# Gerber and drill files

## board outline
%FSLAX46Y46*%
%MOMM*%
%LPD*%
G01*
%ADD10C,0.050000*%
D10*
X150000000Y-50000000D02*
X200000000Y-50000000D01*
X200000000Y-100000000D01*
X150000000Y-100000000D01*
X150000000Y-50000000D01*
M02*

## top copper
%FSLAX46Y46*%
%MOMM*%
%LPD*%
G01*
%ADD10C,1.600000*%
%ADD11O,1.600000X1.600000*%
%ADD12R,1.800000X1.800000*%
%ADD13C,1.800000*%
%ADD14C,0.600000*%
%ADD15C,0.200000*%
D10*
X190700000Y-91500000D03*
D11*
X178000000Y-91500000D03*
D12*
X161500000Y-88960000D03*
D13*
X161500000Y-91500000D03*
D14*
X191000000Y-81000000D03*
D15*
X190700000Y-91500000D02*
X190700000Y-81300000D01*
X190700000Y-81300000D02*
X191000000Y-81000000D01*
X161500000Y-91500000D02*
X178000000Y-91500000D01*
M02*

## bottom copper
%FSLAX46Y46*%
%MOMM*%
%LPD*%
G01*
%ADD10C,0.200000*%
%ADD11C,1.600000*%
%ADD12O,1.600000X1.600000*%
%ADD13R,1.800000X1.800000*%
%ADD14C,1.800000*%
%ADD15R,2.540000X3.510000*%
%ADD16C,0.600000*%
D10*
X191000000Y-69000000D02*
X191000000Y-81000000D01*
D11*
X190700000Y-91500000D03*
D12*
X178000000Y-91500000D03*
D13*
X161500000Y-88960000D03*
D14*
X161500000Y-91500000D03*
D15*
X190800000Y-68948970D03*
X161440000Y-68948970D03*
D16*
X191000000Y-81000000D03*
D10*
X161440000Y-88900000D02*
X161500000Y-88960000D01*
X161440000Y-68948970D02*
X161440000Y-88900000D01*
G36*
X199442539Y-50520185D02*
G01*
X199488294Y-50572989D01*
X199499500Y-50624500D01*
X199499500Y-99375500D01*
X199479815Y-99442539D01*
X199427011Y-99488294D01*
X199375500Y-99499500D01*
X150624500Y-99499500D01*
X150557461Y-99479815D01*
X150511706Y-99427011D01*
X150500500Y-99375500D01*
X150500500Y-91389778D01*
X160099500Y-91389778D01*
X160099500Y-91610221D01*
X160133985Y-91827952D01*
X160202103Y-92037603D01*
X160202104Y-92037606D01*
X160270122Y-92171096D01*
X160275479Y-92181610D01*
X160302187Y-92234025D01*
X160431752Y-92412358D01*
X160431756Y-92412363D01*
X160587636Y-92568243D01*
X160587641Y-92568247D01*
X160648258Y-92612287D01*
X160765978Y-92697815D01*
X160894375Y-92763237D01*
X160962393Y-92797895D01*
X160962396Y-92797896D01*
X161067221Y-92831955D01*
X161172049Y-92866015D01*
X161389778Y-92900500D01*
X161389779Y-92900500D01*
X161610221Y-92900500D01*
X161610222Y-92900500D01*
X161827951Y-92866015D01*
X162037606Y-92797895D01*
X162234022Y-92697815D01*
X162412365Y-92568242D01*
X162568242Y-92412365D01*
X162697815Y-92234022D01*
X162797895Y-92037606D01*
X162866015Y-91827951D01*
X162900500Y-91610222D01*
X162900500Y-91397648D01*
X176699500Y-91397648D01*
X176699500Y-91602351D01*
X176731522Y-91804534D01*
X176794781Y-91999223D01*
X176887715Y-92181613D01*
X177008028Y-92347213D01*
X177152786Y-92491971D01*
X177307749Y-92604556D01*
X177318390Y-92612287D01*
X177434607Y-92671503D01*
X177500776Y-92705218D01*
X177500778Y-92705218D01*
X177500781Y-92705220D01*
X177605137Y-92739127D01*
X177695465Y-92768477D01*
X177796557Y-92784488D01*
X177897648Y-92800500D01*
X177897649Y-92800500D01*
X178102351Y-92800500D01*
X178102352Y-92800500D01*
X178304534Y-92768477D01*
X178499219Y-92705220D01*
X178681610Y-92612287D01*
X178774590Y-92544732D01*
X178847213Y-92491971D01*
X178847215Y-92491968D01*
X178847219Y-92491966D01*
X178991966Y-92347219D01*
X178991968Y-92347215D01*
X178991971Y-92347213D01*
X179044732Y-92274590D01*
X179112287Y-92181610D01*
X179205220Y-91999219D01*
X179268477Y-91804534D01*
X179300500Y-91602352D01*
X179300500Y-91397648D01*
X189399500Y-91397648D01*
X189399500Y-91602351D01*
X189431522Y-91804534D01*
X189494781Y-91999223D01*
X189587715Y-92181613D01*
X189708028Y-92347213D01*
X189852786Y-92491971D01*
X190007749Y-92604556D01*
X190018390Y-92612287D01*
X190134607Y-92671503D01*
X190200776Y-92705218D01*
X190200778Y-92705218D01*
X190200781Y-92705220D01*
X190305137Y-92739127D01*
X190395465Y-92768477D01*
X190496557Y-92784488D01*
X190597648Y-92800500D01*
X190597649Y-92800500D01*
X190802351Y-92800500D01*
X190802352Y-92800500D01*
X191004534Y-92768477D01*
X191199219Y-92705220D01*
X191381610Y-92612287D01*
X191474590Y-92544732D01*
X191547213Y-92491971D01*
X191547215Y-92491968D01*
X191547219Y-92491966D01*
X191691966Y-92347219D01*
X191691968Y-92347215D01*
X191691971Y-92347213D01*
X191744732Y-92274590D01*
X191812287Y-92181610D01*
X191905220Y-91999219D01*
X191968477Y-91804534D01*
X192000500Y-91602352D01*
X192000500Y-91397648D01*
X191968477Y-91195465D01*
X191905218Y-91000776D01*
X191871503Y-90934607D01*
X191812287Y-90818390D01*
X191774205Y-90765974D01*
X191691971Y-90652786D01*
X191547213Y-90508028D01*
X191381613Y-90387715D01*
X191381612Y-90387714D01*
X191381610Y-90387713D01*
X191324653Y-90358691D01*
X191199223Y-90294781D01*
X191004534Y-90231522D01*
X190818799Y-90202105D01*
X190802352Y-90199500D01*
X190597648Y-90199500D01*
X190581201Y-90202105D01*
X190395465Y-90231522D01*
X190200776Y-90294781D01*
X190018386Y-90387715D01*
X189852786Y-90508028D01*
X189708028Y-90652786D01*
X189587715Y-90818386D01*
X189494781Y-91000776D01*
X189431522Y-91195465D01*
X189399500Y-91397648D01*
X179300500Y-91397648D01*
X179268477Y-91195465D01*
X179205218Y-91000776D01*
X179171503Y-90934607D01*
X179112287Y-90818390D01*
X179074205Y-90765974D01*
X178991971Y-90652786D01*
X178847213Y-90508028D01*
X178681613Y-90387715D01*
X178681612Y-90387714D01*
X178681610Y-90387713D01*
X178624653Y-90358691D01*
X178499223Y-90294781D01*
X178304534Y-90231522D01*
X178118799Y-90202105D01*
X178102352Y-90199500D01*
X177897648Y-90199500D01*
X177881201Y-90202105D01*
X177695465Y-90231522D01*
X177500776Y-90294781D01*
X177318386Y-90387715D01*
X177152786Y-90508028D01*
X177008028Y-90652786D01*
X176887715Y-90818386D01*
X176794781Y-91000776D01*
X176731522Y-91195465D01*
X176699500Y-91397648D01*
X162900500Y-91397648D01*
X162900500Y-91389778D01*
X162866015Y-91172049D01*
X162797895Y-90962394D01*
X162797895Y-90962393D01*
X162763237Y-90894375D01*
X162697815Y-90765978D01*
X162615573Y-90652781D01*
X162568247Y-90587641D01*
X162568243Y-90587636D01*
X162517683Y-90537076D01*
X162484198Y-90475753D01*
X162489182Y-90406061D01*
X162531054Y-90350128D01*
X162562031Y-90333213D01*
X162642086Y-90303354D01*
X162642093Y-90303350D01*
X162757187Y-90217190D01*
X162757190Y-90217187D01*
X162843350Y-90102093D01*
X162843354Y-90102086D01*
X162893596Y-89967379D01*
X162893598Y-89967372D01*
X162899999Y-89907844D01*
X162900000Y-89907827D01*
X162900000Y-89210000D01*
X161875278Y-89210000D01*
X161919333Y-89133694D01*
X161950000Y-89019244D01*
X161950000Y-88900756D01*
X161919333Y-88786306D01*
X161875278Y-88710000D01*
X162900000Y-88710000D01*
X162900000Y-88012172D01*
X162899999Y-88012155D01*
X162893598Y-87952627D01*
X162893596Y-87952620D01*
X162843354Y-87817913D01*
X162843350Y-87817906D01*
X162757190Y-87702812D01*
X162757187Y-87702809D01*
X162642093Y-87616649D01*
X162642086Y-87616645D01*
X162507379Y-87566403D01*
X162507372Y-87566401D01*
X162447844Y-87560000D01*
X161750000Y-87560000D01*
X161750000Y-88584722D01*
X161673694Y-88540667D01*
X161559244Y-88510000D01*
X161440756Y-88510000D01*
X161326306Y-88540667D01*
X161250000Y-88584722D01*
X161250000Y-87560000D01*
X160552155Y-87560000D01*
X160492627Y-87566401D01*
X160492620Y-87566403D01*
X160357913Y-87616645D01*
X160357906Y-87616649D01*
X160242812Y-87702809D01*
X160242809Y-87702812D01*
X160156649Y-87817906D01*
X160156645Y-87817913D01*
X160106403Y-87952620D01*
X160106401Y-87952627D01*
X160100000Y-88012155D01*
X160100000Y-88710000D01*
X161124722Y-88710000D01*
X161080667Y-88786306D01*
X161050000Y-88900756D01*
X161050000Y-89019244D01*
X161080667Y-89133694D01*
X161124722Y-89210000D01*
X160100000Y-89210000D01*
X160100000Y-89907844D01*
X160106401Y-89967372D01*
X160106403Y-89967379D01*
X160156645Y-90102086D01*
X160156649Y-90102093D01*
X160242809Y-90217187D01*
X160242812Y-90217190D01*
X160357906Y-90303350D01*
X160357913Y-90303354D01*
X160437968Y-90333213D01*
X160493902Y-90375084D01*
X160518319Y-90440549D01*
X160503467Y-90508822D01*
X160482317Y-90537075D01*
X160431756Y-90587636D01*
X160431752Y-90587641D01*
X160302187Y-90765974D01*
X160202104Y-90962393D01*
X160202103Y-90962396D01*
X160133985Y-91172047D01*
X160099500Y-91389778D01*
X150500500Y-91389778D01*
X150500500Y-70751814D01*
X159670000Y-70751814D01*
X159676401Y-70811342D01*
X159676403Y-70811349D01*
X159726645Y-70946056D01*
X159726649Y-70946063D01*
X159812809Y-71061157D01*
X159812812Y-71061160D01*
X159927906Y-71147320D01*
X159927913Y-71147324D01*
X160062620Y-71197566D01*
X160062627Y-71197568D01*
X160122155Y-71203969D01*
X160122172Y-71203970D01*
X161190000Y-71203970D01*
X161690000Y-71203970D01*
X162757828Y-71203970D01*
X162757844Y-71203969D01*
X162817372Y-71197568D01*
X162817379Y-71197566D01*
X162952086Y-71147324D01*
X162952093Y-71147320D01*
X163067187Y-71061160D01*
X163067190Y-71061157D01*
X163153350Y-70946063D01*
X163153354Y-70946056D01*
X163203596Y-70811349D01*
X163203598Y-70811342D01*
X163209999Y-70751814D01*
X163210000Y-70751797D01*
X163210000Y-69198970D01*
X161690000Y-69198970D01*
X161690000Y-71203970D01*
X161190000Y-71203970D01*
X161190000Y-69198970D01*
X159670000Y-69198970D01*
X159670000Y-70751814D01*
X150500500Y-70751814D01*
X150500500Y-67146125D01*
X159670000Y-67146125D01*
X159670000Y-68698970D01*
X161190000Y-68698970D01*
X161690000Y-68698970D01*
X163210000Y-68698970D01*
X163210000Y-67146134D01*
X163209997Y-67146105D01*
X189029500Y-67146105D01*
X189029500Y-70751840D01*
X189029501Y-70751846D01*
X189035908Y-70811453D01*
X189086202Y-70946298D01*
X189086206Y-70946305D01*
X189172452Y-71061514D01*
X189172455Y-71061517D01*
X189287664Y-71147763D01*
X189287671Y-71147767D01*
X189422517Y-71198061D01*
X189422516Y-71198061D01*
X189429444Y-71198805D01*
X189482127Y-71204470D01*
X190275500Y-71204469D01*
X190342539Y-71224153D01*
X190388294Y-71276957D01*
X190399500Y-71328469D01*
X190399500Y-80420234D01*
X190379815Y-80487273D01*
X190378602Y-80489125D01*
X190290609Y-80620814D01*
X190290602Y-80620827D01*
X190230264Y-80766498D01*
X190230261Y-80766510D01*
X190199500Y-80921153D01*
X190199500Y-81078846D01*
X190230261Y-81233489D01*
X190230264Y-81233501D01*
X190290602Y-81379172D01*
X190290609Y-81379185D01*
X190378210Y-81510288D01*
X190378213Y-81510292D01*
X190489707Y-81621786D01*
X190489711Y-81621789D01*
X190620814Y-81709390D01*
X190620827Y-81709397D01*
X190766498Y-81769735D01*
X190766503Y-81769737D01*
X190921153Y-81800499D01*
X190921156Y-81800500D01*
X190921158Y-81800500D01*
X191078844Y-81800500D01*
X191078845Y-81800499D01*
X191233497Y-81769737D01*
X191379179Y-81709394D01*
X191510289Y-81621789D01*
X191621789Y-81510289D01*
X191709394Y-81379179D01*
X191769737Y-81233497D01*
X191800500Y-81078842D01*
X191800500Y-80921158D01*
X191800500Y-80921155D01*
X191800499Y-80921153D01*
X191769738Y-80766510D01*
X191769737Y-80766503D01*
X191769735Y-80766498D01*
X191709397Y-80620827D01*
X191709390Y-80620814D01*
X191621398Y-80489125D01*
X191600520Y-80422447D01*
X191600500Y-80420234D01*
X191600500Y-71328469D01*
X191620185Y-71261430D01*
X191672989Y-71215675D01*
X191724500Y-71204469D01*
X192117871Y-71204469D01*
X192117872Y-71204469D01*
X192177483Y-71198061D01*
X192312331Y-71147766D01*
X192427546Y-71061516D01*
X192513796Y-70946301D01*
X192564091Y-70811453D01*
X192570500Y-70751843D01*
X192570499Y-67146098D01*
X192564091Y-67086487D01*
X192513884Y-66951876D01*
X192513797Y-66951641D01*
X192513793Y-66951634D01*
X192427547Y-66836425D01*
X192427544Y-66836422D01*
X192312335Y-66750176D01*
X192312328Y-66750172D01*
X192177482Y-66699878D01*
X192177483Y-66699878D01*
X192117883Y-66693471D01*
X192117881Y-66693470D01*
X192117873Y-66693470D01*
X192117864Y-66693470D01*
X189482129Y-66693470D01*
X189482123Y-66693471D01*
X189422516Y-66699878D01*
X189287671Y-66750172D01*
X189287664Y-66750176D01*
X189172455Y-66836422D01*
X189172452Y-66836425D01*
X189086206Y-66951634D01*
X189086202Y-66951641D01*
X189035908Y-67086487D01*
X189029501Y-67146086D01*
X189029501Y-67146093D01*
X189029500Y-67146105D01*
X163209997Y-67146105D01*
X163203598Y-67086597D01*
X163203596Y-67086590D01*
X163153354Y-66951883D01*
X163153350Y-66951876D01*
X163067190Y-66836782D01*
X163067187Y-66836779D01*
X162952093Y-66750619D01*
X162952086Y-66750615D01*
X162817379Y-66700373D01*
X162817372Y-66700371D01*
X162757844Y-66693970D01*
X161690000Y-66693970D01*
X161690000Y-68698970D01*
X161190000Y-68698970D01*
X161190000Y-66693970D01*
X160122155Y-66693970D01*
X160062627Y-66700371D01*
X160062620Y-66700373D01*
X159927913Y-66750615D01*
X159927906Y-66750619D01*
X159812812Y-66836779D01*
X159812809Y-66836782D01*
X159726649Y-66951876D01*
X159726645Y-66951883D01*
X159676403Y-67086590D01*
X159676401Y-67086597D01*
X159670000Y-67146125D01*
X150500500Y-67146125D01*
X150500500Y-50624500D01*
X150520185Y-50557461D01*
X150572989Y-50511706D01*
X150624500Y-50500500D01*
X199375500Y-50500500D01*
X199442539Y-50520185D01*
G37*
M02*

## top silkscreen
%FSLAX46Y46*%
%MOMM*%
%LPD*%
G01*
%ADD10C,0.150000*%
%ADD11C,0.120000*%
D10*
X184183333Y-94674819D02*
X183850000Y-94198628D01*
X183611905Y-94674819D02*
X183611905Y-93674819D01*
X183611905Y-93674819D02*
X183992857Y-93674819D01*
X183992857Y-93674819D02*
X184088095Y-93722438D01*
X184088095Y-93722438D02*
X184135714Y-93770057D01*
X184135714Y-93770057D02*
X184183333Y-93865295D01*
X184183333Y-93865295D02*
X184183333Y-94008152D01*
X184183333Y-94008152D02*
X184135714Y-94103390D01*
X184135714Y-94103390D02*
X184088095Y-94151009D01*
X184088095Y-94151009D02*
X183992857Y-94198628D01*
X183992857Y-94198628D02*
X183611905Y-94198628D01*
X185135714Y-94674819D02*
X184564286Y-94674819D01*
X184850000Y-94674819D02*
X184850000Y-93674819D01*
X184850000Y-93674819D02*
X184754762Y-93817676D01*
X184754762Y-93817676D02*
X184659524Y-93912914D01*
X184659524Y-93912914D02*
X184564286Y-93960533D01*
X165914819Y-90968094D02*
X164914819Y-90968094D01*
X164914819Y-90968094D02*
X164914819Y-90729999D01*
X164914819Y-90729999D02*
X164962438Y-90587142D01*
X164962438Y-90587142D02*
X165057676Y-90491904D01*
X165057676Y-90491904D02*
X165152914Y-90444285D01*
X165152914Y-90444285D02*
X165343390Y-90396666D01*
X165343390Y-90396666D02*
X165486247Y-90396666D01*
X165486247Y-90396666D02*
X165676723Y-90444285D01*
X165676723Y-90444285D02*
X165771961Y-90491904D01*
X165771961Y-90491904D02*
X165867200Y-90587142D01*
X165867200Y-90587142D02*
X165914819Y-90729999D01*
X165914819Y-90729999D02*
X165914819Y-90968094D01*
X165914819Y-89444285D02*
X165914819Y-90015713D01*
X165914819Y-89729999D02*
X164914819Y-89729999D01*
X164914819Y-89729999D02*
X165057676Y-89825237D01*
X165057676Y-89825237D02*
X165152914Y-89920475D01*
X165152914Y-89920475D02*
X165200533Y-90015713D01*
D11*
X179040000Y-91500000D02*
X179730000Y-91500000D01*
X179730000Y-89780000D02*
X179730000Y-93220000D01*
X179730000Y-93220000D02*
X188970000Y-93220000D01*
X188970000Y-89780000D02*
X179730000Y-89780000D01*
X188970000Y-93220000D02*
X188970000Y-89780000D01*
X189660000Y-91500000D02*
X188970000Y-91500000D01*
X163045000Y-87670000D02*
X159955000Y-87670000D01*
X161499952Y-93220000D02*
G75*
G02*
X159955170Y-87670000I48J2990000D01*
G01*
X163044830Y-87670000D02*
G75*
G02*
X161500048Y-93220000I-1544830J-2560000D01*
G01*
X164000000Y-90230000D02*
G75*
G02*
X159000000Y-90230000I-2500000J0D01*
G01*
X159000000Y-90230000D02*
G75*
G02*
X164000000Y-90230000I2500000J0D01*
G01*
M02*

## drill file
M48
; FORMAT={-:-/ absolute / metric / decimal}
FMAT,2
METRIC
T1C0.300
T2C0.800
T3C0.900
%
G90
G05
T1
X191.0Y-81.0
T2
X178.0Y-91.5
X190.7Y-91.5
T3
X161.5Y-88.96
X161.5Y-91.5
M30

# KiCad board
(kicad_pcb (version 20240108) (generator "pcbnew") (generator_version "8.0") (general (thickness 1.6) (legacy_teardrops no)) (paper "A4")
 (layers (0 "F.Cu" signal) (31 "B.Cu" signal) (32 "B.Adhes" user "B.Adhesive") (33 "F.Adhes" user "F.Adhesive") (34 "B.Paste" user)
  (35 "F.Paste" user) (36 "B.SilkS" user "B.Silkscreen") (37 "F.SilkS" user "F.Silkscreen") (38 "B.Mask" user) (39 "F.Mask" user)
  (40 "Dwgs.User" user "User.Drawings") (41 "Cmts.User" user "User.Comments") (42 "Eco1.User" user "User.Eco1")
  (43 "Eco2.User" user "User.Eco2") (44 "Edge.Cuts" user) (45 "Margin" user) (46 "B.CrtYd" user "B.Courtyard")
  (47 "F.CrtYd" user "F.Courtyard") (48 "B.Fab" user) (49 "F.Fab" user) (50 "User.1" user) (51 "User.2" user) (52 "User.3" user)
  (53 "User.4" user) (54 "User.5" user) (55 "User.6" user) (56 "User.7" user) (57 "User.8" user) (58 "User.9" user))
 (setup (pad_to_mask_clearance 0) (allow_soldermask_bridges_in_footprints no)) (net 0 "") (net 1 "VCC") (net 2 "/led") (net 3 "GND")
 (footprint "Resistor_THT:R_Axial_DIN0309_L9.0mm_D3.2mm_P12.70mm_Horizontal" (layer "F.Cu") (at 190.7 91.5 180)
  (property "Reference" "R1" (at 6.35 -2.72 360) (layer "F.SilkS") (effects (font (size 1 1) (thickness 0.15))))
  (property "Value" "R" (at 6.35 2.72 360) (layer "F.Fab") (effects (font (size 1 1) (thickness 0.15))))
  (fp_line (start 11.66 0) (end 10.97 0) (stroke (width 0.12) (type solid)) (layer "F.SilkS"))
  (fp_line (start 10.97 1.72) (end 10.97 -1.72) (stroke (width 0.12) (type solid)) (layer "F.SilkS"))
  (fp_line (start 10.97 -1.72) (end 1.73 -1.72) (stroke (width 0.12) (type solid)) (layer "F.SilkS"))
  (fp_line (start 1.73 1.72) (end 10.97 1.72) (stroke (width 0.12) (type solid)) (layer "F.SilkS"))
  (fp_line (start 1.73 -1.72) (end 1.73 1.72) (stroke (width 0.12) (type solid)) (layer "F.SilkS"))
  (fp_line (start 1.04 0) (end 1.73 0) (stroke (width 0.12) (type solid)) (layer "F.SilkS"))
  (pad "1" thru_hole circle (at 0 0 180) (size 1.6 1.6) (drill 0.8) (layers "*.Cu" "*.Mask") (remove_unused_layers no) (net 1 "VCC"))
  (pad "2" thru_hole oval (at 12.7 0 180) (size 1.6 1.6) (drill 0.8) (layers "*.Cu" "*.Mask") (remove_unused_layers no) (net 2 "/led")))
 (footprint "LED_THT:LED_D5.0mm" (layer "F.Cu") (at 161.5 88.96 -90)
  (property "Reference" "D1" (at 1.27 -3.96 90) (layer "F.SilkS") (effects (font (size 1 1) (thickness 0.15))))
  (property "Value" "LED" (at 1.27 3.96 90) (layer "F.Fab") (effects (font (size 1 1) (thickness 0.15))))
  (fp_line (start -1.29 -1.545) (end -1.29 1.545) (stroke (width 0.12) (type solid)) (layer "F.SilkS"))
  (fp_arc (start 4.26 0.000048) (mid 2.071756 2.880501) (end -1.29 1.54483) (stroke (width 0.12) (type solid)) (layer "F.SilkS"))
  (fp_arc (start -1.29 -1.54483) (mid 2.071756 -2.880501) (end 4.26 -0.000048) (stroke (width 0.12) (type solid)) (layer "F.SilkS"))
  (fp_circle (center 1.27 0) (end 3.77 0) (stroke (width 0.12) (type solid)) (fill none) (layer "F.SilkS"))
  (pad "1" thru_hole rect (at 0 0 270) (size 1.8 1.8) (drill 0.9) (layers "*.Cu" "*.Mask") (remove_unused_layers no) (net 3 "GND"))
  (pad "2" thru_hole circle (at 2.54 0 270) (size 1.8 1.8) (drill 0.9) (layers "*.Cu" "*.Mask") (remove_unused_layers no) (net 2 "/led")))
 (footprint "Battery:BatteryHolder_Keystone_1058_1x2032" (layer "B.Cu") (at 176.12 68.94897 180)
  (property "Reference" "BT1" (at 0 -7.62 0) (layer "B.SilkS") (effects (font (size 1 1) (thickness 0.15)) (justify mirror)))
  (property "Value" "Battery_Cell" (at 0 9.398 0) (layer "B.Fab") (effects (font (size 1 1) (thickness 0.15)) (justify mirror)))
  (pad "1" smd rect (at -14.68 0 180) (size 2.54 3.51) (layers "B.Cu" "B.Paste" "B.Mask") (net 1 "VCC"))
  (pad "2" smd rect (at 14.68 0 180) (size 2.54 3.51) (layers "B.Cu" "B.Paste" "B.Mask") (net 3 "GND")))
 (gr_line (start 191 69) (end 191 81) (stroke (width 0.2) (type default)) (layer "B.Cu") (net 1))
 (gr_rect (start 150 50) (end 200 100) (stroke (width 0.05) (type default)) (fill none) (layer "Edge.Cuts"))
 (segment (start 190.7 91.5) (end 190.7 81.3) (width 0.2) (layer "F.Cu") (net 1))
 (segment (start 190.7 81.3) (end 191 81) (width 0.2) (layer "F.Cu") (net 1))
 (via (at 191 81) (size 0.6) (drill 0.3) (layers "F.Cu" "B.Cu") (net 1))
 (segment (start 161.44 88.9) (end 161.5 88.96) (width 0.2) (layer "B.Cu") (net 3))
 (segment (start 161.44 68.94897) (end 161.44 88.9) (width 0.2) (layer "B.Cu") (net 3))
 (segment (start 161.5 91.5) (end 178 91.5) (width 0.2) (layer "F.Cu") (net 2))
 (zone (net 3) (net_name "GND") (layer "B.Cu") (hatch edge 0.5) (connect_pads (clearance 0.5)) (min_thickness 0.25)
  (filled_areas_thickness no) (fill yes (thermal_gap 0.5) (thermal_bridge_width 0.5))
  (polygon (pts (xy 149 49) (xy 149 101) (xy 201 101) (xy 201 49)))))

